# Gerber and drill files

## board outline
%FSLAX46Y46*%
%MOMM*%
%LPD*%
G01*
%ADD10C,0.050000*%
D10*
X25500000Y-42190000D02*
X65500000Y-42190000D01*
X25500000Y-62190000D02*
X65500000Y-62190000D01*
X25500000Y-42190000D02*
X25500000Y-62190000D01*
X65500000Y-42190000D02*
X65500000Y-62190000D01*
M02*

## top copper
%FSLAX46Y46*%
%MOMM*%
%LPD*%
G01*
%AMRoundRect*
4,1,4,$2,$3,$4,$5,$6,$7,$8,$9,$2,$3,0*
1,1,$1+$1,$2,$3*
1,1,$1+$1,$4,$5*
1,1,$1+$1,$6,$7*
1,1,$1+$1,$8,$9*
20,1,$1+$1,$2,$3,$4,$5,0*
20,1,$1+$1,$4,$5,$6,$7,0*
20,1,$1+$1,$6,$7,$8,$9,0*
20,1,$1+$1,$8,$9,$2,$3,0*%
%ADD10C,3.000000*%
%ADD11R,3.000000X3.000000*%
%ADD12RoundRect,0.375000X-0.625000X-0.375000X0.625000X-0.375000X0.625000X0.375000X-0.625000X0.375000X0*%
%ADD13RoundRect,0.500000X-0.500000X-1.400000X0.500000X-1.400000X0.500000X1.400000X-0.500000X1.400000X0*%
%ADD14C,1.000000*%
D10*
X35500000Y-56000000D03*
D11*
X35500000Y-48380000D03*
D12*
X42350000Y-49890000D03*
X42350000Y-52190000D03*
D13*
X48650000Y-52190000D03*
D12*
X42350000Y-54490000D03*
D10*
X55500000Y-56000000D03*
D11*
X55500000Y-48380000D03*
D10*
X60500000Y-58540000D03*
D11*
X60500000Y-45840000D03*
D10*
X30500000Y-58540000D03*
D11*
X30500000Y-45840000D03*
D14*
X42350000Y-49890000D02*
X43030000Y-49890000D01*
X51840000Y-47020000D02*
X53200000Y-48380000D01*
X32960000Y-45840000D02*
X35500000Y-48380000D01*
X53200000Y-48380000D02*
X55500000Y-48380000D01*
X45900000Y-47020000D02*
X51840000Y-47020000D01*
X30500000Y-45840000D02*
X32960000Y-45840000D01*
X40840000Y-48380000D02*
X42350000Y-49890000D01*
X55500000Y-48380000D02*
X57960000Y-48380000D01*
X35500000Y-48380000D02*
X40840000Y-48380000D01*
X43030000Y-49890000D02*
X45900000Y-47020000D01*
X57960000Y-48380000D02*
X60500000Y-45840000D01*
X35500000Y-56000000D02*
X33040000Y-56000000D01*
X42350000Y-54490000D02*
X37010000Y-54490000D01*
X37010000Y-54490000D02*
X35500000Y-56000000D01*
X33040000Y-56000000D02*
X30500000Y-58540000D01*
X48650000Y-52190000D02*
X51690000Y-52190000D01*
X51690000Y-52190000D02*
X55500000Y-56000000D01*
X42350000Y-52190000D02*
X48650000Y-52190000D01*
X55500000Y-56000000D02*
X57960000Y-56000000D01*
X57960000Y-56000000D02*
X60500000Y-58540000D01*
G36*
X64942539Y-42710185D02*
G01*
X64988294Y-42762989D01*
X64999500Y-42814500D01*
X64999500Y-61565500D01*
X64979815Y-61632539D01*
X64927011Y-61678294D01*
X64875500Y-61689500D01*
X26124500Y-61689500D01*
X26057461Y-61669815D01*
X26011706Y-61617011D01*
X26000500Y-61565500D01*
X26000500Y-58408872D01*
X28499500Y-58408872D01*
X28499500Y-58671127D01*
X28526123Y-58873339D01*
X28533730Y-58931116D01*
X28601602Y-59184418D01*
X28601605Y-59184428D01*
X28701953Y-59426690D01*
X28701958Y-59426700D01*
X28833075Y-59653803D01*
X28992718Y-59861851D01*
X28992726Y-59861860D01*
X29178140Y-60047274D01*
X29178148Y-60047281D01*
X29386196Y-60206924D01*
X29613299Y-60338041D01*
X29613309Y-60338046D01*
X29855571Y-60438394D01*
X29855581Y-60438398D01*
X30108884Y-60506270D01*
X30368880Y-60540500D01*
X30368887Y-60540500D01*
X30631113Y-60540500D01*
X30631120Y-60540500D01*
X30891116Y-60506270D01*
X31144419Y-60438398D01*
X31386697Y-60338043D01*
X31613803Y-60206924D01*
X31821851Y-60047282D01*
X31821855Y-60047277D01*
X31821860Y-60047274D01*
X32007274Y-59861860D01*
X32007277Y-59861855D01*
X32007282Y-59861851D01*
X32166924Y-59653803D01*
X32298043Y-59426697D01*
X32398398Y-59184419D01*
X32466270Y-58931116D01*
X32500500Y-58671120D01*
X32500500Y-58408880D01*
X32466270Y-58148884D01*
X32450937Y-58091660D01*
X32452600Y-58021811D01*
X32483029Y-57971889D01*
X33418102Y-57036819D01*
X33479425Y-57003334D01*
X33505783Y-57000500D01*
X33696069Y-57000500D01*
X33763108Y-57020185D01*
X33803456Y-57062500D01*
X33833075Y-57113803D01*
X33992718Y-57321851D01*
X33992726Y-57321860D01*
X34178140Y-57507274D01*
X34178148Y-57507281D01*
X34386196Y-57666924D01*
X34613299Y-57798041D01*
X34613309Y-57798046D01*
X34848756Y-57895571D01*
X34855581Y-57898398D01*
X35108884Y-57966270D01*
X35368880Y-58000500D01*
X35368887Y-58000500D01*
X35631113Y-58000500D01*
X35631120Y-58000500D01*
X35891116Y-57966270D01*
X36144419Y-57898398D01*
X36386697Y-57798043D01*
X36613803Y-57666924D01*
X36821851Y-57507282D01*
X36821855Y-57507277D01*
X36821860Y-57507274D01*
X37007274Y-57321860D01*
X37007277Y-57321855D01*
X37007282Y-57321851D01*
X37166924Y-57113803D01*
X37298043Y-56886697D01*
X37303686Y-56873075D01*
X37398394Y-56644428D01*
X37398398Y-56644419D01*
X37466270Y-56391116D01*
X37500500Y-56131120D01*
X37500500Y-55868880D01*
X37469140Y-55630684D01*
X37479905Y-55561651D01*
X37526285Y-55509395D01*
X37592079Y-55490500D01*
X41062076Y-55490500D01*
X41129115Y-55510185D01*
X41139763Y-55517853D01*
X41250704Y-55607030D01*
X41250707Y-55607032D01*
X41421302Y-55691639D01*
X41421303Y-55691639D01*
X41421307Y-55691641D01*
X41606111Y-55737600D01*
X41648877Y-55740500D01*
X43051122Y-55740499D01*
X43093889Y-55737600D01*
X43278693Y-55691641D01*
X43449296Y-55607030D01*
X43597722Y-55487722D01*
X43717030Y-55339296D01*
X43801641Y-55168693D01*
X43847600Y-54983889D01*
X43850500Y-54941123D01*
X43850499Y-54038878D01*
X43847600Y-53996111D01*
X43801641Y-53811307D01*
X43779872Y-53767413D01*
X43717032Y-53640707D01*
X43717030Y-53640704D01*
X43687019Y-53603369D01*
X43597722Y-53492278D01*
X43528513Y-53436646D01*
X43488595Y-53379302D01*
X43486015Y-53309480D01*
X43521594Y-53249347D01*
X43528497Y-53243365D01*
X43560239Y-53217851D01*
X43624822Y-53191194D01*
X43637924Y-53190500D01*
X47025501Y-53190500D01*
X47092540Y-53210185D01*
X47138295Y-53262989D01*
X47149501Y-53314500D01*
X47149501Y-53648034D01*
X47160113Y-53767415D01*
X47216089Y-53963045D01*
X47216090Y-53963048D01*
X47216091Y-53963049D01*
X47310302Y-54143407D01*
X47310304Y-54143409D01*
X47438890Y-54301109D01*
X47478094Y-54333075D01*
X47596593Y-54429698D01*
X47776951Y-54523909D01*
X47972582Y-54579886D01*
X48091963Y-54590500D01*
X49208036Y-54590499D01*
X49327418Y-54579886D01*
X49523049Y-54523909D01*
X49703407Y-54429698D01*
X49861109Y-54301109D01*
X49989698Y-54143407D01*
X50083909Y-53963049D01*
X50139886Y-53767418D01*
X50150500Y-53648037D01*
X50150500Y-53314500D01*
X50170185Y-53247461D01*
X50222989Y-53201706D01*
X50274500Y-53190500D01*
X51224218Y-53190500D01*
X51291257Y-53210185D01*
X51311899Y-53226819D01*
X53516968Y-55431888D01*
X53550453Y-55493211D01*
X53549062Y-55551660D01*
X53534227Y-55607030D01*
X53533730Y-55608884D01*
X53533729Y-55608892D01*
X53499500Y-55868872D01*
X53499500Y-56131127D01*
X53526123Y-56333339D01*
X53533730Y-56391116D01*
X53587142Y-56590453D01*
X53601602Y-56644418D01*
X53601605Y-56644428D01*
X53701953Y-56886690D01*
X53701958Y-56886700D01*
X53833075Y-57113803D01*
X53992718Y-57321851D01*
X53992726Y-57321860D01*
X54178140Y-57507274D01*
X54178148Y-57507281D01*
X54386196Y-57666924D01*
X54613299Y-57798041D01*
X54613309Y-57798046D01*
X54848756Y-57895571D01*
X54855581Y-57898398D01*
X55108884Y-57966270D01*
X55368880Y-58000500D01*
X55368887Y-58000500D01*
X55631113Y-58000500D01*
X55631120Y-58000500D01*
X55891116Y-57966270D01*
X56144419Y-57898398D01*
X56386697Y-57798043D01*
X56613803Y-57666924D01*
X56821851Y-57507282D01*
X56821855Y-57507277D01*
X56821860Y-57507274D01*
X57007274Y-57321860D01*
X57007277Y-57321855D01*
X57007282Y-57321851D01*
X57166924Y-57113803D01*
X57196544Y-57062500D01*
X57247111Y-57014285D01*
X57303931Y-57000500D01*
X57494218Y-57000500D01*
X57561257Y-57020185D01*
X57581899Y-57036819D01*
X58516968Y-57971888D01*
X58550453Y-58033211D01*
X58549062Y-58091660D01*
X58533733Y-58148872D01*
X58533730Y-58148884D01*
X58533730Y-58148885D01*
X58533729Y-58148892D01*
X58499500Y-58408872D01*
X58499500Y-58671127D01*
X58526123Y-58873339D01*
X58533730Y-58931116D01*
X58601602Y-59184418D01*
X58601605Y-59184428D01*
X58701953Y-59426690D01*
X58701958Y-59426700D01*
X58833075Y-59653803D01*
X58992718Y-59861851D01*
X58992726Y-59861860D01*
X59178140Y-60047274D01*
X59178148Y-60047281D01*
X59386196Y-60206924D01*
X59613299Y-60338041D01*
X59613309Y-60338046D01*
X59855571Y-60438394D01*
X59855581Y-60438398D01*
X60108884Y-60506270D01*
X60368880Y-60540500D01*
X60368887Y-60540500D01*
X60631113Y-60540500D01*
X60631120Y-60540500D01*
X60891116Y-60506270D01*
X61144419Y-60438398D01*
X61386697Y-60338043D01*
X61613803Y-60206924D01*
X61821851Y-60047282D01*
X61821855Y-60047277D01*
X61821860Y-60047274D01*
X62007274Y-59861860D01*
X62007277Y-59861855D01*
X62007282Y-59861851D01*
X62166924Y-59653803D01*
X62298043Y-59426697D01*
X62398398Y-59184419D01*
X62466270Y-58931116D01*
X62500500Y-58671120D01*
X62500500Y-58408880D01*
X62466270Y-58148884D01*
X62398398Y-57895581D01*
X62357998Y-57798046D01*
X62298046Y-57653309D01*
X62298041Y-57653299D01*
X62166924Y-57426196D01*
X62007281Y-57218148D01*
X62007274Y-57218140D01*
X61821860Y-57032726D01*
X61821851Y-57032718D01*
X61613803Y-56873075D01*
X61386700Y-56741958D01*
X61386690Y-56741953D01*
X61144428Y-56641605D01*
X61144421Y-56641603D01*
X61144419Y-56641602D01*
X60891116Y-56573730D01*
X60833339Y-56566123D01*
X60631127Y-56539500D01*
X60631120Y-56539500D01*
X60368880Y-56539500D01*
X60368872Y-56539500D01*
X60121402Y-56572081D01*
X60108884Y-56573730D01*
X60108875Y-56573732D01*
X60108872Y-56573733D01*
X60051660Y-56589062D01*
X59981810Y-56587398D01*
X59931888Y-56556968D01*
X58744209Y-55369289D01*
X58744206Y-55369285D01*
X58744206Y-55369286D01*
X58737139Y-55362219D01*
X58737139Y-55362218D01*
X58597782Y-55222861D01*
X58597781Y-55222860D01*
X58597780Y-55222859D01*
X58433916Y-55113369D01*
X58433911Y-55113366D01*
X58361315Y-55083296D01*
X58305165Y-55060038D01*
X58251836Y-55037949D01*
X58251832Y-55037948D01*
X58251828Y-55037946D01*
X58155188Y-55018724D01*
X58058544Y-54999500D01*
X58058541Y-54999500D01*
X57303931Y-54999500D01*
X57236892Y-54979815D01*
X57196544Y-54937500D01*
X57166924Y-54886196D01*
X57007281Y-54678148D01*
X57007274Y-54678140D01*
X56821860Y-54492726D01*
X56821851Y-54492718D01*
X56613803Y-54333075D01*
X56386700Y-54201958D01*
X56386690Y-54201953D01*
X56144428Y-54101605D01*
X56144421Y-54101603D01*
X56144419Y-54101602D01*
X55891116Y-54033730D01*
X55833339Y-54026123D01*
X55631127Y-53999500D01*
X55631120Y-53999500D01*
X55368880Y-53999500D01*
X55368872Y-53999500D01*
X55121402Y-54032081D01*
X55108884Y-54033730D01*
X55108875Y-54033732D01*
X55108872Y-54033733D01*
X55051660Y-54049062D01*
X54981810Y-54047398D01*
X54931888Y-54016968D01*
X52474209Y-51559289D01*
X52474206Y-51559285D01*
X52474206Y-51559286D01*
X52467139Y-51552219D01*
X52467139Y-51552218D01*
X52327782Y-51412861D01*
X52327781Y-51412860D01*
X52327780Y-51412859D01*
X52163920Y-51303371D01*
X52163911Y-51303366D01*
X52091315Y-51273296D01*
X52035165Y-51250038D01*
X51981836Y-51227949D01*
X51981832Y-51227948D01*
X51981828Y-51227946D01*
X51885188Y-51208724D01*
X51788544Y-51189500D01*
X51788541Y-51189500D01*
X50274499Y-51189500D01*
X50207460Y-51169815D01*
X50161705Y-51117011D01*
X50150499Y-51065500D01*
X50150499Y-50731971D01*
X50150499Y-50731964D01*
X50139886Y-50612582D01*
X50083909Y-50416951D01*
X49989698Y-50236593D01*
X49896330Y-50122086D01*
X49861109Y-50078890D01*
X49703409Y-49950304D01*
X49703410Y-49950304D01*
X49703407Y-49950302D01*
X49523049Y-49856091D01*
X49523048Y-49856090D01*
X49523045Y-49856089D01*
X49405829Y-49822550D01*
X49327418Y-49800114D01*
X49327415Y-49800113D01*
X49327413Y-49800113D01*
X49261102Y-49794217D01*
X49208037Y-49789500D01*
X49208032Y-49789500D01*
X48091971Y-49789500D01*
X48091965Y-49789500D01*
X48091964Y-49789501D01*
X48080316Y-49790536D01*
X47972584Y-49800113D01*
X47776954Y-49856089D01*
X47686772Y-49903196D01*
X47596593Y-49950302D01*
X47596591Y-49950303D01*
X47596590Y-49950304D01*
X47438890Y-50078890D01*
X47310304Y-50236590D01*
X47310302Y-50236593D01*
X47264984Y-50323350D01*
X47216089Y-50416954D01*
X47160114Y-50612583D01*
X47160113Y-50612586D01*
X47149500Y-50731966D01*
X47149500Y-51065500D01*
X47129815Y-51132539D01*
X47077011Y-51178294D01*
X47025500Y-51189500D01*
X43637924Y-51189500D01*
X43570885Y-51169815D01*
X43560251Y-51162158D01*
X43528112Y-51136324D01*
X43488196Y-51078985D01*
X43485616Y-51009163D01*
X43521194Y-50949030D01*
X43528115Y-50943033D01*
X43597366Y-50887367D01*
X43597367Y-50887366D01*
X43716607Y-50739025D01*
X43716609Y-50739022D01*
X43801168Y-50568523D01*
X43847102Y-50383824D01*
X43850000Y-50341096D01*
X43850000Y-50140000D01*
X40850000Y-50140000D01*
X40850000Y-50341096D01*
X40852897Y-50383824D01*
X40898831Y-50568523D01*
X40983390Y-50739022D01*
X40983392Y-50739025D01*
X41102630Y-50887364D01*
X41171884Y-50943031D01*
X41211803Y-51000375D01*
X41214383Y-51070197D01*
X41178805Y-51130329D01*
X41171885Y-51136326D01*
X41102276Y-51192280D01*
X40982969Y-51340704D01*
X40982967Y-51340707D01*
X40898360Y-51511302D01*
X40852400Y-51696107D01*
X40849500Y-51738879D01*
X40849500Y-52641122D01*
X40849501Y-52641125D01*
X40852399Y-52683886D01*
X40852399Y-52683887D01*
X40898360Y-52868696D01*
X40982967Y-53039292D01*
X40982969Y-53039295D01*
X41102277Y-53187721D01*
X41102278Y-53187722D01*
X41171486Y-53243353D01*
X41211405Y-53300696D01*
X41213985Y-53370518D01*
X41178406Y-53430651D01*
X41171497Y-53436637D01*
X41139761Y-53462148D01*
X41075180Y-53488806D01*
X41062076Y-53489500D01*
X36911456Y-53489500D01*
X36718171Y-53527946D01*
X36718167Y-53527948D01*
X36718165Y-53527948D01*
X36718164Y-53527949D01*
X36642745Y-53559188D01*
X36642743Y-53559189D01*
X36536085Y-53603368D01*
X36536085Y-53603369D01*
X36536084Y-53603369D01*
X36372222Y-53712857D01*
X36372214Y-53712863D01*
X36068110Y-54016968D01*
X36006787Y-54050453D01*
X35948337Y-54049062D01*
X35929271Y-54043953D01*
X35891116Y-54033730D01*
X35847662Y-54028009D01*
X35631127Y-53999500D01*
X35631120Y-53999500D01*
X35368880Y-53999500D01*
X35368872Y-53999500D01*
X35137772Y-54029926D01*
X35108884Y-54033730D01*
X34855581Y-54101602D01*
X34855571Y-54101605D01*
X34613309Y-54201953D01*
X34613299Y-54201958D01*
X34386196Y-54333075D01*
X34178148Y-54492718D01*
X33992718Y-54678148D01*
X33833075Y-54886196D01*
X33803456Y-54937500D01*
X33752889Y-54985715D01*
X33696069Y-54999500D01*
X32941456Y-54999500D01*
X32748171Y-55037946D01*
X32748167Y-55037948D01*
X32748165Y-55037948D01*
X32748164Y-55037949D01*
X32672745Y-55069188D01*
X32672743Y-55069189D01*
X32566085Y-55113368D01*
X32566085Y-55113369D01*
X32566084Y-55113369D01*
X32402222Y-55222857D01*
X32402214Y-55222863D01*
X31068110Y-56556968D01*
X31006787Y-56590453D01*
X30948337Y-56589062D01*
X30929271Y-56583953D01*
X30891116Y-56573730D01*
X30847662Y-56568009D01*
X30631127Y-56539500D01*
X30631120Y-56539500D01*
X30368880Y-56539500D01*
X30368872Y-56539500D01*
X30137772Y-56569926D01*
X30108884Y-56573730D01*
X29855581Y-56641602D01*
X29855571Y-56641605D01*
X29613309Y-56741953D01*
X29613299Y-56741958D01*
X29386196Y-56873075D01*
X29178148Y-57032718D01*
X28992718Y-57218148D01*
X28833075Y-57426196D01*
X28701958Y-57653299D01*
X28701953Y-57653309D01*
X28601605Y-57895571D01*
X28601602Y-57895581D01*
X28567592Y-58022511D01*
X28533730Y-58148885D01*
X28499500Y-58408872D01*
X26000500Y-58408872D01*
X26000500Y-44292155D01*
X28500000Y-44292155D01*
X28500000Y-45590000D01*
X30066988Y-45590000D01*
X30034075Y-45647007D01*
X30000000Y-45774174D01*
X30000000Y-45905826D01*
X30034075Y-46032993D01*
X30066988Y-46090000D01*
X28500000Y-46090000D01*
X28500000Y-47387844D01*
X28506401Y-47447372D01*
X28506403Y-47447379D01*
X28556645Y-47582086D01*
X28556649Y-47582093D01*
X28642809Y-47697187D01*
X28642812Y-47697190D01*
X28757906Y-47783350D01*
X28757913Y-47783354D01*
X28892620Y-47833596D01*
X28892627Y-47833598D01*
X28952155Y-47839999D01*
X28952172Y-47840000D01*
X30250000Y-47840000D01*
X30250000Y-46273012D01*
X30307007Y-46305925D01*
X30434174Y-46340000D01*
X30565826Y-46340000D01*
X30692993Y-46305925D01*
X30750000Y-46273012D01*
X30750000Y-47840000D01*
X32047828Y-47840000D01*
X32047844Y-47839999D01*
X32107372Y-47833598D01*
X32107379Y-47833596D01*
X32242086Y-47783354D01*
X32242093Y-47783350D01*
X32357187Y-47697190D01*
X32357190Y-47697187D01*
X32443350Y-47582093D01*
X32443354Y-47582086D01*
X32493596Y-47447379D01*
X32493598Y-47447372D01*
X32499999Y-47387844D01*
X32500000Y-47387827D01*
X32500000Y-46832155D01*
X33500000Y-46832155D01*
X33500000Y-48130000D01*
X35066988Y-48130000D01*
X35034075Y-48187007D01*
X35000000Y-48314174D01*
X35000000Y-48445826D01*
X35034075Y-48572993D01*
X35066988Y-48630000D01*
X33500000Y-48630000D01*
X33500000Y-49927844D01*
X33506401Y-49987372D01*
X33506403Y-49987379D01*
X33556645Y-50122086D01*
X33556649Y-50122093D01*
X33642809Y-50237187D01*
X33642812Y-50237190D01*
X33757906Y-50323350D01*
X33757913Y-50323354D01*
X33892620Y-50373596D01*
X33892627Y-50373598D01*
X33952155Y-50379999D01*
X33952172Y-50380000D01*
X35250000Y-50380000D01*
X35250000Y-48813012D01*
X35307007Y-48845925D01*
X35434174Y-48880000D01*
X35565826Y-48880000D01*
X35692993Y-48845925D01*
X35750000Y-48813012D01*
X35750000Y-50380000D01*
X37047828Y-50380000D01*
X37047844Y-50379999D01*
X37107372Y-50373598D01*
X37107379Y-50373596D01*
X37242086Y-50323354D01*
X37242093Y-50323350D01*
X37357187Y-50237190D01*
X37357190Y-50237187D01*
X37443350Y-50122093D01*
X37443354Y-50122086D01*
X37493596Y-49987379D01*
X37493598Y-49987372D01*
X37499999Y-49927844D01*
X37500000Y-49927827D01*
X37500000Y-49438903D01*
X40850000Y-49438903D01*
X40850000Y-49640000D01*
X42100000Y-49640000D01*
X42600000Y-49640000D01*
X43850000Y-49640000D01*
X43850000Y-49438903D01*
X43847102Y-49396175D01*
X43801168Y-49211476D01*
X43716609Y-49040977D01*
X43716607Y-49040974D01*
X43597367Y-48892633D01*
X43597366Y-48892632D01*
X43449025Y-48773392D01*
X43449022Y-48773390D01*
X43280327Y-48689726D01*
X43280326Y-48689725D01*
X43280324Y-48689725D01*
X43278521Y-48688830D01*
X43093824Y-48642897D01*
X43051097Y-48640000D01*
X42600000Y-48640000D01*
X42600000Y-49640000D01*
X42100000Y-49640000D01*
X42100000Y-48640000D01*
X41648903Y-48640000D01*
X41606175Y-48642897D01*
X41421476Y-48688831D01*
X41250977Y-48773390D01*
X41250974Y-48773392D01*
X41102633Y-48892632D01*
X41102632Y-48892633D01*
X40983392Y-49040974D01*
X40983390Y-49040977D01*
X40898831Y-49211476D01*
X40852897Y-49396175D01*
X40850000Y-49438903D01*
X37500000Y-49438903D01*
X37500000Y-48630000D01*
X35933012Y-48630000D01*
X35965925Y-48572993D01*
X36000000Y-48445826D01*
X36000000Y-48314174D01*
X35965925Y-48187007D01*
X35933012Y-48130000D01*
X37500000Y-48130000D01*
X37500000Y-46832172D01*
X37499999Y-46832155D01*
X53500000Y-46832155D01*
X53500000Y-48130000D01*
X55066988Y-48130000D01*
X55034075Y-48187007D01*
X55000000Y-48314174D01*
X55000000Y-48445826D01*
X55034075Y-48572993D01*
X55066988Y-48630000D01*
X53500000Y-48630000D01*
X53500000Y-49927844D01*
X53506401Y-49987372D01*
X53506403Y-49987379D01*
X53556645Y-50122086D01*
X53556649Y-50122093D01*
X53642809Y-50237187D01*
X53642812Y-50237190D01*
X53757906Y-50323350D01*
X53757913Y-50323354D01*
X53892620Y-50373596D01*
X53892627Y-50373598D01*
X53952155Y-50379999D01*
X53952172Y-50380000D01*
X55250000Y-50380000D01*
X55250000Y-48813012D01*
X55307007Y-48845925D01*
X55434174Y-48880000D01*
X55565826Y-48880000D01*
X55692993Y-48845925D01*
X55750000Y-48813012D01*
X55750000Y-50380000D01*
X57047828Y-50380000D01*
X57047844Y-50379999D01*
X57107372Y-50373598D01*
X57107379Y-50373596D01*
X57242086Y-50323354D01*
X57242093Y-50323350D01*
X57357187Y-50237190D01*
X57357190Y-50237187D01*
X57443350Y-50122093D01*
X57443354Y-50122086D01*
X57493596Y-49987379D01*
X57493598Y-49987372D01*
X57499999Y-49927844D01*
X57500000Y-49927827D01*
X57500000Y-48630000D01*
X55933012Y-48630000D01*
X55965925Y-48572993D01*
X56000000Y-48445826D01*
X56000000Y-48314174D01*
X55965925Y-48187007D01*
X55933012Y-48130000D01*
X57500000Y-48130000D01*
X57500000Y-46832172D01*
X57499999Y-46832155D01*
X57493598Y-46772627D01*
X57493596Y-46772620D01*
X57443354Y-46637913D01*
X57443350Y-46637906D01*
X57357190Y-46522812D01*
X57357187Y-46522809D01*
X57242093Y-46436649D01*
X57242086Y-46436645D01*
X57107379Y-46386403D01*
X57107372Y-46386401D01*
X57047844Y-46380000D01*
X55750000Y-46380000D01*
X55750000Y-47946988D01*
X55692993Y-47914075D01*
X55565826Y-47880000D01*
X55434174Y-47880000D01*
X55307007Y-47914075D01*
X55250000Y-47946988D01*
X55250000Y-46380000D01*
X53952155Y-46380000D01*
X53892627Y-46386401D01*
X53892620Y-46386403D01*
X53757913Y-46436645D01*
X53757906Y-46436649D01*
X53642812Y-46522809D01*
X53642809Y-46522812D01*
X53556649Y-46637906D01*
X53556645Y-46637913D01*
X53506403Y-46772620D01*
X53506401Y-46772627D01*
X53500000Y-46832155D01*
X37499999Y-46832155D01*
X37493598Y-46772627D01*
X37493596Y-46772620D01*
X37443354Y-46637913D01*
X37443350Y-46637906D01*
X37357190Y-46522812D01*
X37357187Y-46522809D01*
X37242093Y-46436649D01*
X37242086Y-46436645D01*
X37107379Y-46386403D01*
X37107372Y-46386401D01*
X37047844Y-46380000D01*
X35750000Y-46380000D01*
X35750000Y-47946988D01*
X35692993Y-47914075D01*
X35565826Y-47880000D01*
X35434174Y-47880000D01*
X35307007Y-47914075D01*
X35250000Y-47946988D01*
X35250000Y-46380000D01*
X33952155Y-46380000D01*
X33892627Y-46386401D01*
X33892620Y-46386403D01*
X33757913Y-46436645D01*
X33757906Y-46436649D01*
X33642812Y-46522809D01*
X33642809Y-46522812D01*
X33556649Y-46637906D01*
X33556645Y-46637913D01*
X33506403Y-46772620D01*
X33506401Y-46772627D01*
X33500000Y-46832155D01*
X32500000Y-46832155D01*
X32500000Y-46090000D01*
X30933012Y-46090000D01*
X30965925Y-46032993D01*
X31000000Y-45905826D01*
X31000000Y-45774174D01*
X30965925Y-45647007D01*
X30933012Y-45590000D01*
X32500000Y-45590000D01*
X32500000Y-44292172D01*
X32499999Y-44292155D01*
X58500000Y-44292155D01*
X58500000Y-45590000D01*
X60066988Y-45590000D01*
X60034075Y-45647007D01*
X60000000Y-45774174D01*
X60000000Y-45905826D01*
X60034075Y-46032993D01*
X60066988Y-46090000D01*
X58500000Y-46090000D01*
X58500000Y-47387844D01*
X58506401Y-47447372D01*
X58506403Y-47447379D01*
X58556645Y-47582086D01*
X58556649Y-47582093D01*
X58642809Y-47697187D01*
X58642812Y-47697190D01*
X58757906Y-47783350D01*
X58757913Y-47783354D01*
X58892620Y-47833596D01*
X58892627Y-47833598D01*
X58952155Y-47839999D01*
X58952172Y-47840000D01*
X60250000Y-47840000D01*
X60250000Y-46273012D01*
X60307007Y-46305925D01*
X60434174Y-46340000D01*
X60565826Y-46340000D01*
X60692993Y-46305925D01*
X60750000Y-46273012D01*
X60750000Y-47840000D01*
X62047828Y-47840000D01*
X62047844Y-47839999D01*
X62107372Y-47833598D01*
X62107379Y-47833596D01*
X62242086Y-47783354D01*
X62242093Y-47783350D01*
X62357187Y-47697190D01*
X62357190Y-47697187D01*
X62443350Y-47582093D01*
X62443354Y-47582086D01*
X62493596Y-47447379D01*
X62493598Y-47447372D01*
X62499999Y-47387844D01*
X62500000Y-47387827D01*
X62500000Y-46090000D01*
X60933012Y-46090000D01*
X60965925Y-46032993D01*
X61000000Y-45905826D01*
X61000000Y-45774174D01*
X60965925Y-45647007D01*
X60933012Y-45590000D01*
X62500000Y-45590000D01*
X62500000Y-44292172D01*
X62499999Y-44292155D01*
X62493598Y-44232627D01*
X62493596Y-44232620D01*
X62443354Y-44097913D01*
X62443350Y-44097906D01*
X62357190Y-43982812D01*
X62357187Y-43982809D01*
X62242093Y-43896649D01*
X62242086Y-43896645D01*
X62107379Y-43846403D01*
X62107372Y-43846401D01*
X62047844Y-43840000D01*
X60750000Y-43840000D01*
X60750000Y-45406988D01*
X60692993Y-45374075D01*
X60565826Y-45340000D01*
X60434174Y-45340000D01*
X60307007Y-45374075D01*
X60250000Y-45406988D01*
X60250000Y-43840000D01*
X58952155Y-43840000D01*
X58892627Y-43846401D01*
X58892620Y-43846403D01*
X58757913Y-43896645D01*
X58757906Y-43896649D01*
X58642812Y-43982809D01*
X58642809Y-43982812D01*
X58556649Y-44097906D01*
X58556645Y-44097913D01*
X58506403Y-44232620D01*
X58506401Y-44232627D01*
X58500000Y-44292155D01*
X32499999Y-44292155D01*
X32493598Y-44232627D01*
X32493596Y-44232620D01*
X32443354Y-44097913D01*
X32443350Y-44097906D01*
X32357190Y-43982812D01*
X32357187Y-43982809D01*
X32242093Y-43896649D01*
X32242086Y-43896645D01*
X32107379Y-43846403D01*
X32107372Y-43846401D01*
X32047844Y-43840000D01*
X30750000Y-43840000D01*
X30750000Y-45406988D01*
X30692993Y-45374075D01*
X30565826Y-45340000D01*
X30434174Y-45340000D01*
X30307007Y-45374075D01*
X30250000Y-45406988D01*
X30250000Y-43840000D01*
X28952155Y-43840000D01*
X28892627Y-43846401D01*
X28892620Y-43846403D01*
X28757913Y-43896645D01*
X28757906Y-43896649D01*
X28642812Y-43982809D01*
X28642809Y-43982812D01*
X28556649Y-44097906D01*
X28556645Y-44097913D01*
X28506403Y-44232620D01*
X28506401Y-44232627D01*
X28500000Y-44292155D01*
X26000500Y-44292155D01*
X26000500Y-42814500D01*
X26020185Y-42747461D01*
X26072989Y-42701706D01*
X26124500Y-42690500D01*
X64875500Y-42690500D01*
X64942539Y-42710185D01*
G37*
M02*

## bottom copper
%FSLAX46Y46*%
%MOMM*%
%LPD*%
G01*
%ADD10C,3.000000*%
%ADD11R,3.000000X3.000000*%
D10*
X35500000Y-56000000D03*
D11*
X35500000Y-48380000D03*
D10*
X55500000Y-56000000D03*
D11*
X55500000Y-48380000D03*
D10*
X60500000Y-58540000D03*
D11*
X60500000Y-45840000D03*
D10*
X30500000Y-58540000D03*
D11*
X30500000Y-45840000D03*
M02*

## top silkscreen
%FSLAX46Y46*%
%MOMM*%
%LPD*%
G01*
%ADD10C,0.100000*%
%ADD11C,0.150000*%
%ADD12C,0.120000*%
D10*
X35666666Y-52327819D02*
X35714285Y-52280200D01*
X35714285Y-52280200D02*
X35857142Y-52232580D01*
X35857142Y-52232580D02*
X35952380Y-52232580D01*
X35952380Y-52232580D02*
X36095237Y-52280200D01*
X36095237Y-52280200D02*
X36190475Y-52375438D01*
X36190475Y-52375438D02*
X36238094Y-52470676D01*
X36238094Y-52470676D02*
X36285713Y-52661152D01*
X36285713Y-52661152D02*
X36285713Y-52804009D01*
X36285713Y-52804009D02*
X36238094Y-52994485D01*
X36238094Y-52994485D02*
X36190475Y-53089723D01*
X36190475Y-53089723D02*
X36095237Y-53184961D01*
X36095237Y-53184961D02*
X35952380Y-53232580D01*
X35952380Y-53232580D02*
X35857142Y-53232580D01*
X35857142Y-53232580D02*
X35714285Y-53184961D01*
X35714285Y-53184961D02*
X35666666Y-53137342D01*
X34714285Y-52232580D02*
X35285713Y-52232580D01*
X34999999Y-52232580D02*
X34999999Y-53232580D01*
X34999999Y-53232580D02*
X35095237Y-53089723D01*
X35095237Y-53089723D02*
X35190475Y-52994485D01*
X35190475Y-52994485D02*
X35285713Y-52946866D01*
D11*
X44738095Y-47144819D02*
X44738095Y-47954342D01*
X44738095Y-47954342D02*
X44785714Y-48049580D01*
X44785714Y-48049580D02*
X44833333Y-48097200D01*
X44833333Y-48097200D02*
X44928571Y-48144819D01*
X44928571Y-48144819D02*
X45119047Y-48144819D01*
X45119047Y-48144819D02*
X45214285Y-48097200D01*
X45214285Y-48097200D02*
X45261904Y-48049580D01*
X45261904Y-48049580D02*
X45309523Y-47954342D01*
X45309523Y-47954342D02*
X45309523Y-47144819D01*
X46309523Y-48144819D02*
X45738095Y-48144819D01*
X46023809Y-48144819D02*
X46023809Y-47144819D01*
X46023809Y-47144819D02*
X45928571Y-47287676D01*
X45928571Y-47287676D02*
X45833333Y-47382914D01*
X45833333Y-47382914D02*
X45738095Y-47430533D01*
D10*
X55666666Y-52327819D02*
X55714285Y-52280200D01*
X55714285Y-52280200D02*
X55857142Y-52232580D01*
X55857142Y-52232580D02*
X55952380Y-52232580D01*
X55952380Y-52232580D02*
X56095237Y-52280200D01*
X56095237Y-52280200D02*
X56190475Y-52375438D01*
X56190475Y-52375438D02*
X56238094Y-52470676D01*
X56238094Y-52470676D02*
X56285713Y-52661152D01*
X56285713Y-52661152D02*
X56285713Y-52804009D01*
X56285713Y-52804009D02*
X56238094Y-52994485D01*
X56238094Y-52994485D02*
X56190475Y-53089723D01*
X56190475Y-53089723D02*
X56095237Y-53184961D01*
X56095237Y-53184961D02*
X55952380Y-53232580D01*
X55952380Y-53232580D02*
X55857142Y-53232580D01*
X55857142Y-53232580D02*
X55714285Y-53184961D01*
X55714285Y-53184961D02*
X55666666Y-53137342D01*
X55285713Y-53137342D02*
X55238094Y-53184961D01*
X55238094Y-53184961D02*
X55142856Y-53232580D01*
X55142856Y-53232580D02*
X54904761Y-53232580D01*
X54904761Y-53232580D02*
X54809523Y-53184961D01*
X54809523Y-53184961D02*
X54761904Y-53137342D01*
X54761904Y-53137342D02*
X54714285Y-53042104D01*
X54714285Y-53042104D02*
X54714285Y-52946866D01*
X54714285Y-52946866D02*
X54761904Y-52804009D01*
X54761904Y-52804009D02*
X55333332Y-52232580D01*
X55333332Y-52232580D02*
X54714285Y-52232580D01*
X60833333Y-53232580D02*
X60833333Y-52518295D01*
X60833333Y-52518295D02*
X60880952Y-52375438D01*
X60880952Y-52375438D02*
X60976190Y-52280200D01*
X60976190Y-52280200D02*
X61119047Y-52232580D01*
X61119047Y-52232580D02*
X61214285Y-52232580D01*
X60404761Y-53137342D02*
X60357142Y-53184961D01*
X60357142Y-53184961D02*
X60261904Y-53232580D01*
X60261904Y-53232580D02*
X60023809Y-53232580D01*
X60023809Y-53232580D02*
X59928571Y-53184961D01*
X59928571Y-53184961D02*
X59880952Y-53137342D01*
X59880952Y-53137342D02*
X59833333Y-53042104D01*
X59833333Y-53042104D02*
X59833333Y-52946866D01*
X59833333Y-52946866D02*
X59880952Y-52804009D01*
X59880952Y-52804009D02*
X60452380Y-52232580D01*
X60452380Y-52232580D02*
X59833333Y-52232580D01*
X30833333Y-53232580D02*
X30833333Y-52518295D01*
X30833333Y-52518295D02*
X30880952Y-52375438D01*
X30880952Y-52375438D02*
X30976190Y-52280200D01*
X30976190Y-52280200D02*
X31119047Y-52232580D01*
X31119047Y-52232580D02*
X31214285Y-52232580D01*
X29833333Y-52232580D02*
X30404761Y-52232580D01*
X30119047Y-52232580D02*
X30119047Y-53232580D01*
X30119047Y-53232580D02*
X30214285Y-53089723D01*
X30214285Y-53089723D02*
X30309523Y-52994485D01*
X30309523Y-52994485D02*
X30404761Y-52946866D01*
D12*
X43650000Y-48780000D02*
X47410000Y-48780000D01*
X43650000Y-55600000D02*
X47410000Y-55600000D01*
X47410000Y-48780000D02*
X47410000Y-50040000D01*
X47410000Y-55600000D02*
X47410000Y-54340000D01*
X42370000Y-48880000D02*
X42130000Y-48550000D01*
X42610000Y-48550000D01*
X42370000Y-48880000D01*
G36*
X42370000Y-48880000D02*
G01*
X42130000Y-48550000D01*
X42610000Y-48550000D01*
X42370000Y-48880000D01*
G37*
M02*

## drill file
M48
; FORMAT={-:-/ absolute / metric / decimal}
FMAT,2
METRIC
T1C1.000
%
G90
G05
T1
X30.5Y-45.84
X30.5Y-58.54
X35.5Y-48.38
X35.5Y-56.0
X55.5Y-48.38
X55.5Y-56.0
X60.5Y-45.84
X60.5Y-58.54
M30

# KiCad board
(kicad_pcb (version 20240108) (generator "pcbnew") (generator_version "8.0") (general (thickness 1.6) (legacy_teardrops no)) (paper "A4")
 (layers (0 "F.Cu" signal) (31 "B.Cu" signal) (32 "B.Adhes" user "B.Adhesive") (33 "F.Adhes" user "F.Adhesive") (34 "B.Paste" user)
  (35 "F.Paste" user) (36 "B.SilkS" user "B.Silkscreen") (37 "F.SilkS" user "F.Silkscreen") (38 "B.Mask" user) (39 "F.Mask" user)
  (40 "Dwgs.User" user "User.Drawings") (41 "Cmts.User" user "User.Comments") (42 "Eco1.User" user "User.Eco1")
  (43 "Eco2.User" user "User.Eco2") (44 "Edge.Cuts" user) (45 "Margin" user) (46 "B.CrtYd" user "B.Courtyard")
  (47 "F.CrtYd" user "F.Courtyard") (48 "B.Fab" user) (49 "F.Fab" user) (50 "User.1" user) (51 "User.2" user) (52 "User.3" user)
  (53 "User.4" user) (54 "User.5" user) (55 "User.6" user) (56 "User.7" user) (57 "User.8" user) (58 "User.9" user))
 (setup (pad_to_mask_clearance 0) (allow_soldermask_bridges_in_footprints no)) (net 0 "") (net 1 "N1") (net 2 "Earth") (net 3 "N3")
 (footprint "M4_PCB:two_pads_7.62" (layer "F.Cu") (at 35.5 52.19 180)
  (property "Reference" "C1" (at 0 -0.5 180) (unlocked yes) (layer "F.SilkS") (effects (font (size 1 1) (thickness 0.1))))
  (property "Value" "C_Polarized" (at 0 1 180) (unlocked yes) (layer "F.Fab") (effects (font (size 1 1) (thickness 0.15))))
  (pad "1" thru_hole circle (at 0 -3.81 180) (size 3 3) (drill 1) (layers "*.Cu" "*.Mask") (remove_unused_layers no) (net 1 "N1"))
  (pad "3" thru_hole rect (at 0 3.81 180) (size 3 3) (drill 1) (layers "*.Cu" "*.Mask") (remove_unused_layers no) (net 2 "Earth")))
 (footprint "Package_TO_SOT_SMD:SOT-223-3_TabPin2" (layer "F.Cu") (at 45.5 52.19)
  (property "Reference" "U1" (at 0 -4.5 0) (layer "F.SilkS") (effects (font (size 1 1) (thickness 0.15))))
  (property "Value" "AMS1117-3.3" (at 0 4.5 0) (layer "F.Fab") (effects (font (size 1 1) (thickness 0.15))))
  (fp_line (start -1.85 -3.41) (end 1.91 -3.41) (stroke (width 0.12) (type solid)) (layer "F.SilkS"))
  (fp_line (start -1.85 3.41) (end 1.91 3.41) (stroke (width 0.12) (type solid)) (layer "F.SilkS"))
  (fp_line (start 1.91 -3.41) (end 1.91 -2.15) (stroke (width 0.12) (type solid)) (layer "F.SilkS"))
  (fp_line (start 1.91 3.41) (end 1.91 2.15) (stroke (width 0.12) (type solid)) (layer "F.SilkS"))
  (fp_poly
   (pts (xy -3.13 -3.31) (xy -3.37 -3.64) (xy -2.89 -3.64) (xy -3.13 -3.31)) (stroke (width 0.12) (type solid)) (fill solid)
   (layer "F.SilkS"))
  (pad "1" smd roundrect (at -3.15 -2.3) (size 2 1.5) (layers "F.Cu" "F.Paste" "F.Mask") (roundrect_rratio 0.25) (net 2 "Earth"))
  (pad "2" smd roundrect (at -3.15 0) (size 2 1.5) (layers "F.Cu" "F.Paste" "F.Mask") (roundrect_rratio 0.25) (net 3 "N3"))
  (pad "2" smd roundrect (at 3.15 0) (size 2 3.8) (layers "F.Cu" "F.Paste" "F.Mask") (roundrect_rratio 0.25) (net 3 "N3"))
  (pad "3" smd roundrect (at -3.15 2.3) (size 2 1.5) (layers "F.Cu" "F.Paste" "F.Mask") (roundrect_rratio 0.25) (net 1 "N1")))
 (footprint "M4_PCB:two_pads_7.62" (layer "F.Cu") (at 55.5 52.19 180)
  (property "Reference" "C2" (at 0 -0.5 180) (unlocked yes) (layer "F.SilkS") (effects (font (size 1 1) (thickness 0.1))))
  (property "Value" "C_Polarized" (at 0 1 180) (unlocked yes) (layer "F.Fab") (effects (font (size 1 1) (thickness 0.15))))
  (pad "1" thru_hole circle (at 0 -3.81 180) (size 3 3) (drill 1) (layers "*.Cu" "*.Mask") (remove_unused_layers no) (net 3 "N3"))
  (pad "2" thru_hole rect (at 0 3.81 180) (size 3 3) (drill 1) (layers "*.Cu" "*.Mask") (remove_unused_layers no) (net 2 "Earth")))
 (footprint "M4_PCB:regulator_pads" (layer "F.Cu") (at 60.5 52.19 180)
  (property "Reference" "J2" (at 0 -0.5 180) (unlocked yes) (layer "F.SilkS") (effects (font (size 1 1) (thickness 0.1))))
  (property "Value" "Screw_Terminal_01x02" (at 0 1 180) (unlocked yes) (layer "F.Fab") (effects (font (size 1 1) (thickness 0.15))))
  (pad "1" thru_hole circle (at 0 -6.35 180) (size 3 3) (drill 1) (layers "*.Cu" "*.Mask") (remove_unused_layers no) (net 3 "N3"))
  (pad "2" thru_hole rect (at 0 6.35 180) (size 3 3) (drill 1) (layers "*.Cu" "*.Mask") (remove_unused_layers no) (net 2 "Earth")))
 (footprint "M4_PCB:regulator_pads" (layer "F.Cu") (at 30.5 52.19 180)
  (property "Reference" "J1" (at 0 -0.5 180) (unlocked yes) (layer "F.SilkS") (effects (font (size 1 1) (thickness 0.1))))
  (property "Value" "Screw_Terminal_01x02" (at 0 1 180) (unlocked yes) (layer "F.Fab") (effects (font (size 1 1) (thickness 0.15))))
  (pad "1" thru_hole circle (at 0 -6.35 180) (size 3 3) (drill 1) (layers "*.Cu" "*.Mask") (remove_unused_layers no) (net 1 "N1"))
  (pad "2" thru_hole rect (at 0 6.35 180) (size 3 3) (drill 1) (layers "*.Cu" "*.Mask") (remove_unused_layers no) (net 2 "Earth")))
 (gr_line (start 25.5 42.19) (end 65.5 42.19) (stroke (width 0.05) (type default)) (layer "Edge.Cuts"))
 (gr_line (start 25.5 62.19) (end 65.5 62.19) (stroke (width 0.05) (type default)) (layer "Edge.Cuts"))
 (gr_line (start 25.5 42.19) (end 25.5 62.19) (stroke (width 0.05) (type default)) (layer "Edge.Cuts"))
 (gr_line (start 65.5 42.19) (end 65.5 62.19) (stroke (width 0.05) (type default)) (layer "Edge.Cuts"))
 (segment (start 42.35 49.89) (end 43.03 49.89) (width 1) (layer "F.Cu") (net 2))
 (segment (start 51.84 47.02) (end 53.2 48.38) (width 1) (layer "F.Cu") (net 2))
 (segment (start 32.96 45.84) (end 35.5 48.38) (width 1) (layer "F.Cu") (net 2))
 (segment (start 53.2 48.38) (end 55.5 48.38) (width 1) (layer "F.Cu") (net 2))
 (segment (start 45.9 47.02) (end 51.84 47.02) (width 1) (layer "F.Cu") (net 2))
 (segment (start 30.5 45.84) (end 32.96 45.84) (width 1) (layer "F.Cu") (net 2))
 (segment (start 40.84 48.38) (end 42.35 49.89) (width 1) (layer "F.Cu") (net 2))
 (segment (start 55.5 48.38) (end 57.96 48.38) (width 1) (layer "F.Cu") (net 2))
 (segment (start 35.5 48.38) (end 40.84 48.38) (width 1) (layer "F.Cu") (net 2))
 (segment (start 43.03 49.89) (end 45.9 47.02) (width 1) (layer "F.Cu") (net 2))
 (segment (start 57.96 48.38) (end 60.5 45.84) (width 1) (layer "F.Cu") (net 2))
 (segment (start 35.5 56) (end 33.04 56) (width 1) (layer "F.Cu") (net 1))
 (segment (start 42.35 54.49) (end 37.01 54.49) (width 1) (layer "F.Cu") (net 1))
 (segment (start 37.01 54.49) (end 35.5 56) (width 1) (layer "F.Cu") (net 1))
 (segment (start 33.04 56) (end 30.5 58.54) (width 1) (layer "F.Cu") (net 1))
 (segment (start 48.65 52.19) (end 51.69 52.19) (width 1) (layer "F.Cu") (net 3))
 (segment (start 51.69 52.19) (end 55.5 56) (width 1) (layer "F.Cu") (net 3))
 (segment (start 42.35 52.19) (end 48.65 52.19) (width 1) (layer "F.Cu") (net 3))
 (segment (start 55.5 56) (end 57.96 56) (width 1) (layer "F.Cu") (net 3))
 (segment (start 57.96 56) (end 60.5 58.54) (width 1) (layer "F.Cu") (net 3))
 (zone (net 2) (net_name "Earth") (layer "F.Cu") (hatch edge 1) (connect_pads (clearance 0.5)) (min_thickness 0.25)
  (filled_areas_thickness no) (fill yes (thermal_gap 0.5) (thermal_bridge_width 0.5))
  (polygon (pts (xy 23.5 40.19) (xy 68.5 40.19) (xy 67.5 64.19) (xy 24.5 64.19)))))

